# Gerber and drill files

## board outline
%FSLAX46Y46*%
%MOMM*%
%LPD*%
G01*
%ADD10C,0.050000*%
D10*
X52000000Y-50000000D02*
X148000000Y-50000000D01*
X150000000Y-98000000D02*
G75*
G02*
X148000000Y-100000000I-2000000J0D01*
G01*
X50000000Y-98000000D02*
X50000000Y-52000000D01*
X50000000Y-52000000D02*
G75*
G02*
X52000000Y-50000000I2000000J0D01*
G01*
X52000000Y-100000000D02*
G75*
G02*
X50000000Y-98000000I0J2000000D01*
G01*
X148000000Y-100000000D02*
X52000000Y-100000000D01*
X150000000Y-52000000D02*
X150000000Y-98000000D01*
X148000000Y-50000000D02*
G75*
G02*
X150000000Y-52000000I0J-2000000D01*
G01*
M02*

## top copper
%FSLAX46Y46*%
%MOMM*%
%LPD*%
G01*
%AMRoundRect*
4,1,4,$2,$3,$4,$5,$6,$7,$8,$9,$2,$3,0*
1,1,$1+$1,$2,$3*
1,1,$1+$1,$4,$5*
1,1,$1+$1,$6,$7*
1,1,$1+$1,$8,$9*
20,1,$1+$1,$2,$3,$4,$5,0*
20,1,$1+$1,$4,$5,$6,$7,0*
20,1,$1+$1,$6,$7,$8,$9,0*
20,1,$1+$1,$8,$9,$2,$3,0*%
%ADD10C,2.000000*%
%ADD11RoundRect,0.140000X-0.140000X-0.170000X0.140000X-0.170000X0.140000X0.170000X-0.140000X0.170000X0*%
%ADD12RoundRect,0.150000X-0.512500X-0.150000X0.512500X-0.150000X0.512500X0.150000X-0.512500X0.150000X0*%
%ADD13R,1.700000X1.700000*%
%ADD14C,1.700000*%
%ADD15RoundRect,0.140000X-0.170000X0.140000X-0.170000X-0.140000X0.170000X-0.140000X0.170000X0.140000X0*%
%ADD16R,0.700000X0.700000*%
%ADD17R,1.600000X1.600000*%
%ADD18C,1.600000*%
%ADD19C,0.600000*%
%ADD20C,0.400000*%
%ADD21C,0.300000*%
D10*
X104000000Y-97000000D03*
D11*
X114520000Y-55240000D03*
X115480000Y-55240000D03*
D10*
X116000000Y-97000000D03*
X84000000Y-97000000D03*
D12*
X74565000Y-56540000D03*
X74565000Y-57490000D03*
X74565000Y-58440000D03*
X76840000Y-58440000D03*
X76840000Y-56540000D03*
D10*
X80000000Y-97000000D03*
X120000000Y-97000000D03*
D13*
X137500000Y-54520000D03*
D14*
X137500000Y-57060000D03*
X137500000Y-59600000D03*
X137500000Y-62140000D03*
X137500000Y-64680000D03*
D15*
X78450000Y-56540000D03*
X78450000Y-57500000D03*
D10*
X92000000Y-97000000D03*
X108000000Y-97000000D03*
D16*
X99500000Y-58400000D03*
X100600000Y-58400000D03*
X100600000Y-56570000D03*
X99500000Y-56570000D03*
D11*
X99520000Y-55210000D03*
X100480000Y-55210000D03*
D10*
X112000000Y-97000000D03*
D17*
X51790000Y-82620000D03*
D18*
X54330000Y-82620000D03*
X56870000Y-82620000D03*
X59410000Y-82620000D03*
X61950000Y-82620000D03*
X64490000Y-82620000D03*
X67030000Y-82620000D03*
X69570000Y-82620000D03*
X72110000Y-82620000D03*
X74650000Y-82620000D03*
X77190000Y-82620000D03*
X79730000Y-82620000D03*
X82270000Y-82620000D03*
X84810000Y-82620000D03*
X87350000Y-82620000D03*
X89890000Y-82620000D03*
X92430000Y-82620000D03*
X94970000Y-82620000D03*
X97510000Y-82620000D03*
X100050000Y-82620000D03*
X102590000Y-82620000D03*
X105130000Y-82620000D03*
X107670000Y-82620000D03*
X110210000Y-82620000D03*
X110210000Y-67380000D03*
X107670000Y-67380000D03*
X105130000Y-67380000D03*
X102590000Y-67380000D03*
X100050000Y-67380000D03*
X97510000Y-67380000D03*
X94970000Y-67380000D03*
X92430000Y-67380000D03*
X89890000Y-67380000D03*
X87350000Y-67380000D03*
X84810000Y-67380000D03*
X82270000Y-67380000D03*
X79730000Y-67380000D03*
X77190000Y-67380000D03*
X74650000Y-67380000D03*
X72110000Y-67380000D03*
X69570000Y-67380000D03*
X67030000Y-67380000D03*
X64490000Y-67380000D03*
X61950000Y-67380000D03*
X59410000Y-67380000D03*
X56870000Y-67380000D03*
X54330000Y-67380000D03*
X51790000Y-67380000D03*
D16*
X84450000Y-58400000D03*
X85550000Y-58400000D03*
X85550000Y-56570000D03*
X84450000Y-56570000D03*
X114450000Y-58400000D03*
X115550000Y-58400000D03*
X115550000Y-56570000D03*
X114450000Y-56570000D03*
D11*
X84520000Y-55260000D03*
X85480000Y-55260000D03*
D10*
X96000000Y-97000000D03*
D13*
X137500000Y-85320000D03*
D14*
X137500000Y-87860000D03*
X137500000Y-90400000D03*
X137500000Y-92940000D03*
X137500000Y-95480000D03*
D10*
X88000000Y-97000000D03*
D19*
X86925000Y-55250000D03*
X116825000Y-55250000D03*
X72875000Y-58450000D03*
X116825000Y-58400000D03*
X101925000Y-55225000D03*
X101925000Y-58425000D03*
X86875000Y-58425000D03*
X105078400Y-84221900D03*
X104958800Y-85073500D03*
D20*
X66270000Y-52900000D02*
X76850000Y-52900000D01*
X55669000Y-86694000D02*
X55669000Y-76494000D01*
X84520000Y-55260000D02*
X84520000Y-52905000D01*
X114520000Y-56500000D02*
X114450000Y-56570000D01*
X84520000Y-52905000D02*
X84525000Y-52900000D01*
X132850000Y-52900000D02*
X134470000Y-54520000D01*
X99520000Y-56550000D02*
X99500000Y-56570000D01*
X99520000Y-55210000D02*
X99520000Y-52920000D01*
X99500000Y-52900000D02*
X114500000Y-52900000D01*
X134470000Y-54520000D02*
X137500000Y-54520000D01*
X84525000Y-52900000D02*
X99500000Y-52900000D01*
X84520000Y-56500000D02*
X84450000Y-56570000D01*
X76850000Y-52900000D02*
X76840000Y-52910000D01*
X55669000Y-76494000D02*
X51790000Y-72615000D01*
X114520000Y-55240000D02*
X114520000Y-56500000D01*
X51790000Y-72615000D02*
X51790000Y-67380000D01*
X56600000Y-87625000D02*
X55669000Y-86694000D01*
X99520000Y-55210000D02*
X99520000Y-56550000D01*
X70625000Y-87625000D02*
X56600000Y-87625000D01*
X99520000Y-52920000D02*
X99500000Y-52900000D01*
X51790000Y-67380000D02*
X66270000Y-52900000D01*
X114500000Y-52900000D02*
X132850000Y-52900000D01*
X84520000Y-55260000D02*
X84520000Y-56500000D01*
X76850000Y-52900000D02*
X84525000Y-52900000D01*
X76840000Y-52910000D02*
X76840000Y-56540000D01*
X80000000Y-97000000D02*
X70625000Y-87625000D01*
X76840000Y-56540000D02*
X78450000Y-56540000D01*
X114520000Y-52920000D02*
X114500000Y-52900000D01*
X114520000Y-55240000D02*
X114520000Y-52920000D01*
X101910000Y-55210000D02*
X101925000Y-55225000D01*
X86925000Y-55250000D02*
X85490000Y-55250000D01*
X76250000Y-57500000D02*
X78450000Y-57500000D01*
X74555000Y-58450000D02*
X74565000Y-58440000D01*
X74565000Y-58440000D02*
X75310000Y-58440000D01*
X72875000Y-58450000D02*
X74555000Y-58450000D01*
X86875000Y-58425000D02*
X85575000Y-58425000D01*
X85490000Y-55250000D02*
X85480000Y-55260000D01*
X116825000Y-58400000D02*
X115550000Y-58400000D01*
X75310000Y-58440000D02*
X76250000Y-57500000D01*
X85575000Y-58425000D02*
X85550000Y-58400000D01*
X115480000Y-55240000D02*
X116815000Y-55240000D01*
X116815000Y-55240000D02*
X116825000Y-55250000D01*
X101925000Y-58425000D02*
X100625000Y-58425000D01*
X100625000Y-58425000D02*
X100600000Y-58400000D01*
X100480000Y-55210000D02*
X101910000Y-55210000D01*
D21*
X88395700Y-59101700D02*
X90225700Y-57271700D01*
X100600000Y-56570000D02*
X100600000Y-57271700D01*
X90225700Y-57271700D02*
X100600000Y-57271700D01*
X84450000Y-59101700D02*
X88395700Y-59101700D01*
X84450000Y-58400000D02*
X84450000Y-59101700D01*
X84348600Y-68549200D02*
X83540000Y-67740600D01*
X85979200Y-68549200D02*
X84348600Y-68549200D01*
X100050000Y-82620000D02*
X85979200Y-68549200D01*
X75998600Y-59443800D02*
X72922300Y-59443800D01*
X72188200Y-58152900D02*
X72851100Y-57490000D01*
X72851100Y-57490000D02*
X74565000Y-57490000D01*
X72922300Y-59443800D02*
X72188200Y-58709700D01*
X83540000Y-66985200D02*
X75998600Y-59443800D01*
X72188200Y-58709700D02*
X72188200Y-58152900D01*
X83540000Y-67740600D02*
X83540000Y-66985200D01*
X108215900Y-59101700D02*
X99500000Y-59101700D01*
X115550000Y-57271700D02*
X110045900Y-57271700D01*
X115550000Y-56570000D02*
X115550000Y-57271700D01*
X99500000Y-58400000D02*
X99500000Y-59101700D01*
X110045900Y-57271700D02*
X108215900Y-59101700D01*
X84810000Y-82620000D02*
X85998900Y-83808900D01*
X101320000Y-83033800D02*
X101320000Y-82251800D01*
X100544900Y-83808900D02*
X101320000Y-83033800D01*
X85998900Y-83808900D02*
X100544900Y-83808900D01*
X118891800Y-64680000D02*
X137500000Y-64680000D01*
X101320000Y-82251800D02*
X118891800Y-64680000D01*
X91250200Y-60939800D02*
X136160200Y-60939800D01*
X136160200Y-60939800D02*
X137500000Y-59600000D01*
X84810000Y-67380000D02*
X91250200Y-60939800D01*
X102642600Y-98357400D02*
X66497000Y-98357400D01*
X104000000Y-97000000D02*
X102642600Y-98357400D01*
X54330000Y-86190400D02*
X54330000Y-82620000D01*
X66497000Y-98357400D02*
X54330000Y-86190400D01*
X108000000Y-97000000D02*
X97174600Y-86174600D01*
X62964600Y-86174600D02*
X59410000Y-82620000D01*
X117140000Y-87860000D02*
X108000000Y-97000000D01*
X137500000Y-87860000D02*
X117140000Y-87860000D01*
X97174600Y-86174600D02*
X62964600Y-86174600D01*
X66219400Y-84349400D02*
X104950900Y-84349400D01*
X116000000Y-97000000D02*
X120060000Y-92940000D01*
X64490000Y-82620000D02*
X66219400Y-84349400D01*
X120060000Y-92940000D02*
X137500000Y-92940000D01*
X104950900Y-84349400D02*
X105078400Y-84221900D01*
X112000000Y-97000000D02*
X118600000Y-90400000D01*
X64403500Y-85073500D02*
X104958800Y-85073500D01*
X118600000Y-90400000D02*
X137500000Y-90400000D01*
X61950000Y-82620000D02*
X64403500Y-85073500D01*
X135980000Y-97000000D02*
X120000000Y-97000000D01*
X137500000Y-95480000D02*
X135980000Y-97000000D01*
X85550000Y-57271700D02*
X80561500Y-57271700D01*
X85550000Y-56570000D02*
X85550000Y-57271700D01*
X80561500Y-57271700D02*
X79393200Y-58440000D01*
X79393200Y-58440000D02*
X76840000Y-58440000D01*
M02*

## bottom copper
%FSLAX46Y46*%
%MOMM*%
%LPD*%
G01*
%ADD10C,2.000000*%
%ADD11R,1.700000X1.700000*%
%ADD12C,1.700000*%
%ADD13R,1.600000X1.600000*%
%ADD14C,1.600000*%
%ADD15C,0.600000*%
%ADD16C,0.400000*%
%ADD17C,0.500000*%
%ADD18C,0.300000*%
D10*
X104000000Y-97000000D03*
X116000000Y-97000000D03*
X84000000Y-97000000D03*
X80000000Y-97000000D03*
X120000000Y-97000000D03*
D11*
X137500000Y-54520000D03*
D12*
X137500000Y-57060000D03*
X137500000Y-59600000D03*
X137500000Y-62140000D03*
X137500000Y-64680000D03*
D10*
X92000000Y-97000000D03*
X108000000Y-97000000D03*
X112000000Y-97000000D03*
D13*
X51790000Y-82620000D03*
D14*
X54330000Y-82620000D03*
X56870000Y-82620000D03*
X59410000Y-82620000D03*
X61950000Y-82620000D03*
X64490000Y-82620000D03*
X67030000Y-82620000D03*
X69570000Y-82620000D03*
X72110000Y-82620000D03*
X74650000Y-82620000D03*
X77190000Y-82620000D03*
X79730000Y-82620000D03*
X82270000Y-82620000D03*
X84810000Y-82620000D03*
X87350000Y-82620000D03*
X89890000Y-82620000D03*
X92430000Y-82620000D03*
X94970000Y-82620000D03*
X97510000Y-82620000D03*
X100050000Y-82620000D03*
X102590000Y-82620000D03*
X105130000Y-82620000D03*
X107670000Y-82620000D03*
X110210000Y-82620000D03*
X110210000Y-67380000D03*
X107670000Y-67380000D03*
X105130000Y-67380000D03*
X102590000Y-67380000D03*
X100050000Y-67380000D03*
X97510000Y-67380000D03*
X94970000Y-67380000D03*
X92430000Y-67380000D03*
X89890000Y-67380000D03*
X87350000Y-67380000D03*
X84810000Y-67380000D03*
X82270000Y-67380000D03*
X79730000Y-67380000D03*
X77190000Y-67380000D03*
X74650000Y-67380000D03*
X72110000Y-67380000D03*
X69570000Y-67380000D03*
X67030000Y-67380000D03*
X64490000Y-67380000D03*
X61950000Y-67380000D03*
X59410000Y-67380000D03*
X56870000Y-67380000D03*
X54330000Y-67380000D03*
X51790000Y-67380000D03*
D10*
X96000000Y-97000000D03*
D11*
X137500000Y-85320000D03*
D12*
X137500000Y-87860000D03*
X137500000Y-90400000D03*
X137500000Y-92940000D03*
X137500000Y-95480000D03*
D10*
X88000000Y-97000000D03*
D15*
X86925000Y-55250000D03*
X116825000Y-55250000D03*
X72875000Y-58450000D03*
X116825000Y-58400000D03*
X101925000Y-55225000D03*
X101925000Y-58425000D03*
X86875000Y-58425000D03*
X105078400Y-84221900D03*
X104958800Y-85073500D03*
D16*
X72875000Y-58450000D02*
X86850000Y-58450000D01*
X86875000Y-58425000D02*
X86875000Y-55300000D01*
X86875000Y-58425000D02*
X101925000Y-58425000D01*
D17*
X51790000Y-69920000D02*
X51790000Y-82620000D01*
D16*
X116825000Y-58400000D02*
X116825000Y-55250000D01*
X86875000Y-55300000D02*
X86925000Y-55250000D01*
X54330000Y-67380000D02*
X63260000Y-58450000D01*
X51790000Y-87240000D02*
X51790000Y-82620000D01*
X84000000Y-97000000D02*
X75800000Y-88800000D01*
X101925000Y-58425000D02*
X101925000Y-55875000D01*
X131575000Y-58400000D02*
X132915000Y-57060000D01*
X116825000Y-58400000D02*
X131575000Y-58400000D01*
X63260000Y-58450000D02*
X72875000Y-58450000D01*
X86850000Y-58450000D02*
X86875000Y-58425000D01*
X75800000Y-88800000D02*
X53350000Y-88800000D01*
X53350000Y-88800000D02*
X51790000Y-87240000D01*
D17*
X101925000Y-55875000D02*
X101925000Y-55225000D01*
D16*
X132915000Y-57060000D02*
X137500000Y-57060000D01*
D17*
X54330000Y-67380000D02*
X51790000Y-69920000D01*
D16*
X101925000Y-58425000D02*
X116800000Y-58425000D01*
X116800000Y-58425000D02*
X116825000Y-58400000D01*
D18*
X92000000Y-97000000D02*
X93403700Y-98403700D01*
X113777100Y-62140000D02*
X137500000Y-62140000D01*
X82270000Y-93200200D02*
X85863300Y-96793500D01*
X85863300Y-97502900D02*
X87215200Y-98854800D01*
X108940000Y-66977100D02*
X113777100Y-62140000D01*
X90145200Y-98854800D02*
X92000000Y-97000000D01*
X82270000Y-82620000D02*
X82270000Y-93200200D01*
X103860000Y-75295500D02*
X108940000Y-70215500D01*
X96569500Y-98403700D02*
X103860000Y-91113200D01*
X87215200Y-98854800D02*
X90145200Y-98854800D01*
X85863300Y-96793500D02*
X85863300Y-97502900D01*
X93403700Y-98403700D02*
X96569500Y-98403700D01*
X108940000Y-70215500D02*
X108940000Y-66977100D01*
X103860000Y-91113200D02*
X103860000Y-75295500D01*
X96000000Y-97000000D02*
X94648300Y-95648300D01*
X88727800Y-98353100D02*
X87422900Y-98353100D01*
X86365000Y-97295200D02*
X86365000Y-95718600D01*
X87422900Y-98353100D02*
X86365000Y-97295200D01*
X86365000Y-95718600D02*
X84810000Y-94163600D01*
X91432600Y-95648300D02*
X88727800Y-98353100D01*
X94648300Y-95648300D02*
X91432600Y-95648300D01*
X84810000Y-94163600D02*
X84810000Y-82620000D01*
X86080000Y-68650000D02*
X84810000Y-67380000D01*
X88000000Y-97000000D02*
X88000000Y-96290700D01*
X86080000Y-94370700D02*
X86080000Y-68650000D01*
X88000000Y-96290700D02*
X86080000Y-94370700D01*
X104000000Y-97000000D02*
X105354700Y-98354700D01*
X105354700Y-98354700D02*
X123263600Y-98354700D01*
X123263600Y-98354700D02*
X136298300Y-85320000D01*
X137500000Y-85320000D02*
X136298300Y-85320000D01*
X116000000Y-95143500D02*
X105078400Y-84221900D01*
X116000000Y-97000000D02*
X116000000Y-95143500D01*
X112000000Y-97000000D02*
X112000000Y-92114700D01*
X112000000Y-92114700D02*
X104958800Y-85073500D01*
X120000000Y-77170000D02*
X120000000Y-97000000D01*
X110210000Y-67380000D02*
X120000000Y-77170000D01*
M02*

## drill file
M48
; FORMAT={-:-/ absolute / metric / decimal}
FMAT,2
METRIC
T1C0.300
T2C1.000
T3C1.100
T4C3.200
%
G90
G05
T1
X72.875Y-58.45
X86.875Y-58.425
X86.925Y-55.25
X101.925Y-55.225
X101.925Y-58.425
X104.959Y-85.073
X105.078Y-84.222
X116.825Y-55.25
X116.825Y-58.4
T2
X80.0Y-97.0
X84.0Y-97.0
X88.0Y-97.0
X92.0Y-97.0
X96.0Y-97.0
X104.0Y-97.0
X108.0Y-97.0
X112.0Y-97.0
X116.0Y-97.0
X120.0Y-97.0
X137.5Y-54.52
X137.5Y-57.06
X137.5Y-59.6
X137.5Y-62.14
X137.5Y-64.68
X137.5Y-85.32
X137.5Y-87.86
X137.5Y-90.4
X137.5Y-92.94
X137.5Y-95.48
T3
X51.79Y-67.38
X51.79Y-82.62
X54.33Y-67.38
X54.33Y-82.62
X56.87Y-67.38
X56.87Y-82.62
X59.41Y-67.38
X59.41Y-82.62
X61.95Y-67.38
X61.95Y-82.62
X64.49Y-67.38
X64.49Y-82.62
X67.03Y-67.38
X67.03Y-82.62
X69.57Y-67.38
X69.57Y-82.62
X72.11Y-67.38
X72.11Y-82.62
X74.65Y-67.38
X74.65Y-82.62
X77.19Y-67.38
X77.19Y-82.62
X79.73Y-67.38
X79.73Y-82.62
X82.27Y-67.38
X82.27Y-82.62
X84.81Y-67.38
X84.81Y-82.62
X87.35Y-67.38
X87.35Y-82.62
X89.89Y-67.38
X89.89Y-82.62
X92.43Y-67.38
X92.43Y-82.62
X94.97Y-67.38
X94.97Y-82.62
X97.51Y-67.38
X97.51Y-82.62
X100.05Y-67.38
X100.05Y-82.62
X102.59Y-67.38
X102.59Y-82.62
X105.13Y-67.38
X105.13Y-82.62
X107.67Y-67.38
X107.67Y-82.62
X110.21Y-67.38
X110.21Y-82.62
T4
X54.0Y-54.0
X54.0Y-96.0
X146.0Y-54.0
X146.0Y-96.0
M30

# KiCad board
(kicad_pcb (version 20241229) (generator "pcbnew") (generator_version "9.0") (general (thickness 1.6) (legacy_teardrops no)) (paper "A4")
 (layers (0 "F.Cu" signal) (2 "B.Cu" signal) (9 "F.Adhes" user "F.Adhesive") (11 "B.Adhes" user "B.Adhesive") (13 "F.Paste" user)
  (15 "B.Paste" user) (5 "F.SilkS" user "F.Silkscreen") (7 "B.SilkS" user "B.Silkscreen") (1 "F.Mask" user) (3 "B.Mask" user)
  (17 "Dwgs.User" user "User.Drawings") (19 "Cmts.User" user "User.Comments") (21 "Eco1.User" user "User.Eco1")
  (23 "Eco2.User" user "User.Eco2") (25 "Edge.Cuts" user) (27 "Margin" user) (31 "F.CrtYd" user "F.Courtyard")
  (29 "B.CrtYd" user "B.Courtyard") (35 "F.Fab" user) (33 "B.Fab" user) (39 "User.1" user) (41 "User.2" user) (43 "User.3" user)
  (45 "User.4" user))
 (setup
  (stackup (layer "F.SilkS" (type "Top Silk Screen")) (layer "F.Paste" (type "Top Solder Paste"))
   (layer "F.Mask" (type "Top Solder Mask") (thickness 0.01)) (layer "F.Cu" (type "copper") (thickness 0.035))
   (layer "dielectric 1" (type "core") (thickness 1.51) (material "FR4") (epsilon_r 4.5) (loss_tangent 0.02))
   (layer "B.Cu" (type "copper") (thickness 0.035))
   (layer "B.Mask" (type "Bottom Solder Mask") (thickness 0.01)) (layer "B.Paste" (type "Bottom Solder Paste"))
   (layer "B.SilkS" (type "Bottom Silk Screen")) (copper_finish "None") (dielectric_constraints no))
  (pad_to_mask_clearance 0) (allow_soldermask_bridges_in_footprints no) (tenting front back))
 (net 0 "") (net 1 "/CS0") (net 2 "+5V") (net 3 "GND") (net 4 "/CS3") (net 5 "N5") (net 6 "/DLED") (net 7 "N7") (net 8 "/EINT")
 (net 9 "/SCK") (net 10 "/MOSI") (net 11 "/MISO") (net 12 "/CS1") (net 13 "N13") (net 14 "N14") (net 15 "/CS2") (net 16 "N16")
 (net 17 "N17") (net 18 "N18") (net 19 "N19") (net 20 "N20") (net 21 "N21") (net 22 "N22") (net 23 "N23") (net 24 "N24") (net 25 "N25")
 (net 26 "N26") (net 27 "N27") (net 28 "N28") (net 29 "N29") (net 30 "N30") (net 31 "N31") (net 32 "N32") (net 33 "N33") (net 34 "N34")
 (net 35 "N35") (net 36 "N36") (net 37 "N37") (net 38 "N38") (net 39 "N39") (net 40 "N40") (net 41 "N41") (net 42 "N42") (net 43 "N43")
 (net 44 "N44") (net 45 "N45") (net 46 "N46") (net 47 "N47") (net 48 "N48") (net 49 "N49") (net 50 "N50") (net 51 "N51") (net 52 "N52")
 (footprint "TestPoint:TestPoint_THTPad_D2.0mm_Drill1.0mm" (layer "F.Cu") (at 104 97 90)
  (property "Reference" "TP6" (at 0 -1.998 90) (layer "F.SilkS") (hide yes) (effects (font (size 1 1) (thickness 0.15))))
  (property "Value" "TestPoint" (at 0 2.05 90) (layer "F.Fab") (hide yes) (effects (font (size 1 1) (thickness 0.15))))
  (pad "1" thru_hole circle (at 0 0 90) (size 2 2) (drill 1) (layers "*.Cu" "*.Mask") (remove_unused_layers no) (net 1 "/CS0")))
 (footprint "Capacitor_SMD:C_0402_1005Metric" (layer "F.Cu") (at 115 55.24)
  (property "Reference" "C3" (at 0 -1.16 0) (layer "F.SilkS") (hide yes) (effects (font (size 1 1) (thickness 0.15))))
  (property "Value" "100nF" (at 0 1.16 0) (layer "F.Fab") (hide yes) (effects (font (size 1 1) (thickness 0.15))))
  (pad "1" smd roundrect (at -0.48 0) (size 0.56 0.62) (layers "F.Cu" "F.Mask" "F.Paste") (roundrect_rratio 0.25) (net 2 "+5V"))
  (pad "2" smd roundrect (at 0.48 0) (size 0.56 0.62) (layers "F.Cu" "F.Mask" "F.Paste") (roundrect_rratio 0.25) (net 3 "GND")))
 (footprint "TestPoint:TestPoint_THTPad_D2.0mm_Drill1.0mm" (layer "F.Cu") (at 116 97 90)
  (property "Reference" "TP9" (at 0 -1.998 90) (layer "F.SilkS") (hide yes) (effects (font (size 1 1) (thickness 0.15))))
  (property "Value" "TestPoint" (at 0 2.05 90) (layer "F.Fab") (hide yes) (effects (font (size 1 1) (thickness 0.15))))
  (pad "1" thru_hole circle (at 0 0 90) (size 2 2) (drill 1) (layers "*.Cu" "*.Mask") (remove_unused_layers no) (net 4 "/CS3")))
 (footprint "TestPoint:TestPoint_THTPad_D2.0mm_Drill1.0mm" (layer "F.Cu") (at 84 97 90)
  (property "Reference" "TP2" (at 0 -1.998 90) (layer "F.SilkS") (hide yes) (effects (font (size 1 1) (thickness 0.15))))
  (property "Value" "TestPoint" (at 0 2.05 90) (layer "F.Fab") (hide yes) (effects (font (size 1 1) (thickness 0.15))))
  (pad "1" thru_hole circle (at 0 0 90) (size 2 2) (drill 1) (layers "*.Cu" "*.Mask") (remove_unused_layers no) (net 3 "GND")))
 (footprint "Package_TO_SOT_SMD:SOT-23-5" (layer "F.Cu") (at 75.7025 57.49)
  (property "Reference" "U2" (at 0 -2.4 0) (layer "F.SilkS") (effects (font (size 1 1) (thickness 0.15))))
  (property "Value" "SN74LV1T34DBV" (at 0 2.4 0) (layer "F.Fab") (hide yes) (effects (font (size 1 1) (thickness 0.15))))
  (pad "1" smd roundrect (at -1.1375 -0.95) (size 1.325 0.6) (layers "F.Cu" "F.Mask" "F.Paste") (roundrect_rratio 0.25) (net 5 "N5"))
  (pad "2" smd roundrect (at -1.1375 0) (size 1.325 0.6) (layers "F.Cu" "F.Mask" "F.Paste") (roundrect_rratio 0.25) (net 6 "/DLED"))
  (pad "3" smd roundrect (at -1.1375 0.95) (size 1.325 0.6) (layers "F.Cu" "F.Mask" "F.Paste") (roundrect_rratio 0.25) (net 3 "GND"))
  (pad "4" smd roundrect (at 1.1375 0.95) (size 1.325 0.6) (layers "F.Cu" "F.Mask" "F.Paste") (roundrect_rratio 0.25) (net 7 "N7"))
  (pad "5" smd roundrect (at 1.1375 -0.95) (size 1.325 0.6) (layers "F.Cu" "F.Mask" "F.Paste") (roundrect_rratio 0.25) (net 2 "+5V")))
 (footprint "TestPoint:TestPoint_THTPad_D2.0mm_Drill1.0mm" (layer "F.Cu") (at 80 97 90)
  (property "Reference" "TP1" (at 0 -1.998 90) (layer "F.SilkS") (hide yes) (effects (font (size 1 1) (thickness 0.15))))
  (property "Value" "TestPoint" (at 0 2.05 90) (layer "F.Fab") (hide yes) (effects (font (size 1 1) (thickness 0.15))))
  (pad "1" thru_hole circle (at 0 0 90) (size 2 2) (drill 1) (layers "*.Cu" "*.Mask") (remove_unused_layers no) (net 2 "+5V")))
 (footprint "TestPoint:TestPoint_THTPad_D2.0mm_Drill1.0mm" (layer "F.Cu") (at 120 97 90)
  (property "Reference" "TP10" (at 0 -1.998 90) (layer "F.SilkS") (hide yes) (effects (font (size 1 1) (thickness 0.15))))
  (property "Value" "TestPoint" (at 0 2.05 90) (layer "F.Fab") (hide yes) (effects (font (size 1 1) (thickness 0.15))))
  (pad "1" thru_hole circle (at 0 0 90) (size 2 2) (drill 1) (layers "*.Cu" "*.Mask") (remove_unused_layers no) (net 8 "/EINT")))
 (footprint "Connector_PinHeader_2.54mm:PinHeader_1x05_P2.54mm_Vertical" (layer "F.Cu") (at 137.5 54.52)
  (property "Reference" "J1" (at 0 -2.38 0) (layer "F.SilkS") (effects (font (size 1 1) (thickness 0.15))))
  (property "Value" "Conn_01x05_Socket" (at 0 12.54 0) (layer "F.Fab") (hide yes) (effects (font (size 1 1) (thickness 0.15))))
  (pad "1" thru_hole rect (at 0 0) (size 1.7 1.7) (drill 1) (layers "*.Cu" "*.Mask") (remove_unused_layers no) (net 2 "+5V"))
  (pad "2" thru_hole circle (at 0 2.54) (size 1.7 1.7) (drill 1) (layers "*.Cu" "*.Mask") (remove_unused_layers no) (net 3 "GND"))
  (pad "3" thru_hole circle (at 0 5.08) (size 1.7 1.7) (drill 1) (layers "*.Cu" "*.Mask") (remove_unused_layers no) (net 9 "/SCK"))
  (pad "4" thru_hole circle (at 0 7.62) (size 1.7 1.7) (drill 1) (layers "*.Cu" "*.Mask") (remove_unused_layers no) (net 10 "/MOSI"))
  (pad "5" thru_hole circle (at 0 10.16) (size 1.7 1.7) (drill 1) (layers "*.Cu" "*.Mask") (remove_unused_layers no) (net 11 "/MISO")))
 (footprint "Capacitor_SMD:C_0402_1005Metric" (layer "F.Cu") (at 78.45 57.02 -90)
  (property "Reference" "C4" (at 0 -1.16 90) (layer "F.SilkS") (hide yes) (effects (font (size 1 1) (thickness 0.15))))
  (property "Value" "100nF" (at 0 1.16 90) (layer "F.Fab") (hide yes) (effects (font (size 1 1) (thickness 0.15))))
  (pad "1" smd roundrect (at -0.48 0 270) (size 0.56 0.62) (layers "F.Cu" "F.Mask" "F.Paste") (roundrect_rratio 0.25) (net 2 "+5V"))
  (pad "2" smd roundrect (at 0.48 0 270) (size 0.56 0.62) (layers "F.Cu" "F.Mask" "F.Paste") (roundrect_rratio 0.25) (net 3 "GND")))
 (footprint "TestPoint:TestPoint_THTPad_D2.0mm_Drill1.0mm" (layer "F.Cu") (at 92 97 90)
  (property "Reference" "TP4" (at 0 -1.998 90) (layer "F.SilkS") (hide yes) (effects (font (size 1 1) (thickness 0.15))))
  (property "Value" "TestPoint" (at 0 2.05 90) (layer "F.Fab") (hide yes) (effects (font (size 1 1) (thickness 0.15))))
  (pad "1" thru_hole circle (at 0 0 90) (size 2 2) (drill 1) (layers "*.Cu" "*.Mask") (remove_unused_layers no) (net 10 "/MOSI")))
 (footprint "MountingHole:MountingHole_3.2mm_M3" (layer "F.Cu") (at 54 96)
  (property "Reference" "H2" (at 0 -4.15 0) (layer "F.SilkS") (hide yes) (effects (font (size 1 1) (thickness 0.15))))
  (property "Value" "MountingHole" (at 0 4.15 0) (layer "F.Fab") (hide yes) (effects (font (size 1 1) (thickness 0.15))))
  (pad "" np_thru_hole circle (at 0 0) (size 3.2 3.2) (drill 3.2) (layers "*.Cu" "*.Mask")))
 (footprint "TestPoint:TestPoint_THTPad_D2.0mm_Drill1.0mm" (layer "F.Cu") (at 108 97 90)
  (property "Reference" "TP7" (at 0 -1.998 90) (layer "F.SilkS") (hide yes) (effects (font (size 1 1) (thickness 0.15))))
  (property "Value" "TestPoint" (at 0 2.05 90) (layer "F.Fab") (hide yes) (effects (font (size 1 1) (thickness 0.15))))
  (pad "1" thru_hole circle (at 0 0 90) (size 2 2) (drill 1) (layers "*.Cu" "*.Mask") (remove_unused_layers no) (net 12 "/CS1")))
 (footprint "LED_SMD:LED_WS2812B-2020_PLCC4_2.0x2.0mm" (layer "F.Cu") (at 100.05 57.485 90)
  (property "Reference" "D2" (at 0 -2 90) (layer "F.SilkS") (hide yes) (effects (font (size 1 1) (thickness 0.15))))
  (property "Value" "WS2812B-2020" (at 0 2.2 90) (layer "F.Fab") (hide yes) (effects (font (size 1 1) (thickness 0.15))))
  (pad "1" smd rect (at -0.915 -0.55 90) (size 0.7 0.7) (layers "F.Cu" "F.Mask" "F.Paste") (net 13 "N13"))
  (pad "2" smd rect (at -0.915 0.55 90) (size 0.7 0.7) (layers "F.Cu" "F.Mask" "F.Paste") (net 3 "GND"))
  (pad "3" smd rect (at 0.915 0.55 90) (size 0.7 0.7) (layers "F.Cu" "F.Mask" "F.Paste") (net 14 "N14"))
  (pad "4" smd rect (at 0.915 -0.55 90) (size 0.7 0.7) (layers "F.Cu" "F.Mask" "F.Paste") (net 2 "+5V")))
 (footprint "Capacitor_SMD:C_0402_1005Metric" (layer "F.Cu") (at 100 55.21)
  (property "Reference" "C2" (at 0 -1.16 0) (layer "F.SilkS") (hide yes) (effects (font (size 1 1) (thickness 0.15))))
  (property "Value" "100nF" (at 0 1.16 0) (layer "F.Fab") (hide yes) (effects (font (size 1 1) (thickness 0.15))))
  (pad "1" smd roundrect (at -0.48 0) (size 0.56 0.62) (layers "F.Cu" "F.Mask" "F.Paste") (roundrect_rratio 0.25) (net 2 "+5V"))
  (pad "2" smd roundrect (at 0.48 0) (size 0.56 0.62) (layers "F.Cu" "F.Mask" "F.Paste") (roundrect_rratio 0.25) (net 3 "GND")))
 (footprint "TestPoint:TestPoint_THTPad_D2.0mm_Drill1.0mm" (layer "F.Cu") (at 112 97 90)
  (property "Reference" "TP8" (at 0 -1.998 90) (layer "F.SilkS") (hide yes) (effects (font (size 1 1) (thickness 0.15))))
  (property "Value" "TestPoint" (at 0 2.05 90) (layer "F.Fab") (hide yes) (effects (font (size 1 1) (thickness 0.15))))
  (pad "1" thru_hole circle (at 0 0 90) (size 2 2) (drill 1) (layers "*.Cu" "*.Mask") (remove_unused_layers no) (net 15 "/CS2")))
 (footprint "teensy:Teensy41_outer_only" (layer "F.Cu") (at 81 75)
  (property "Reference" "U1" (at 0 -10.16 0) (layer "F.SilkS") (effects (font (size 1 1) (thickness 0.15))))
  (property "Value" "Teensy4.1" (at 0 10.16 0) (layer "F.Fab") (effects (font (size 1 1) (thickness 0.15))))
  (pad "1" thru_hole rect (at -29.21 7.62) (size 1.6 1.6) (drill 1.1) (layers "*.Cu" "*.Mask") (remove_unused_layers no) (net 3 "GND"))
  (pad "2" thru_hole circle (at -26.67 7.62) (size 1.6 1.6) (drill 1.1) (layers "*.Cu" "*.Mask") (remove_unused_layers no) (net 1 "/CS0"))
  (pad "3" thru_hole circle (at -24.13 7.62) (size 1.6 1.6) (drill 1.1) (layers "*.Cu" "*.Mask") (remove_unused_layers no) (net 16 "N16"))
  (pad "4" thru_hole circle (at -21.59 7.62) (size 1.6 1.6) (drill 1.1) (layers "*.Cu" "*.Mask") (remove_unused_layers no) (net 12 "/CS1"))
  (pad "5" thru_hole circle (at -19.05 7.62) (size 1.6 1.6) (drill 1.1) (layers "*.Cu" "*.Mask") (remove_unused_layers no) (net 15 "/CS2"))
  (pad "6" thru_hole circle (at -16.51 7.62) (size 1.6 1.6) (drill 1.1) (layers "*.Cu" "*.Mask") (remove_unused_layers no) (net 4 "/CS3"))
  (pad "7" thru_hole circle (at -13.97 7.62) (size 1.6 1.6) (drill 1.1) (layers "*.Cu" "*.Mask") (remove_unused_layers no) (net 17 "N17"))
  (pad "8" thru_hole circle (at -11.43 7.62) (size 1.6 1.6) (drill 1.1) (layers "*.Cu" "*.Mask") (remove_unused_layers no) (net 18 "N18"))
  (pad "9" thru_hole circle (at -8.89 7.62) (size 1.6 1.6) (drill 1.1) (layers "*.Cu" "*.Mask") (remove_unused_layers no) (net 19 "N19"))
  (pad "10" thru_hole circle (at -6.35 7.62) (size 1.6 1.6) (drill 1.1) (layers "*.Cu" "*.Mask") (remove_unused_layers no) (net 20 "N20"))
  (pad "11" thru_hole circle (at -3.81 7.62) (size 1.6 1.6) (drill 1.1) (layers "*.Cu" "*.Mask") (remove_unused_layers no) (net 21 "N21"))
  (pad "12" thru_hole circle (at -1.27 7.62) (size 1.6 1.6) (drill 1.1) (layers "*.Cu" "*.Mask") (remove_unused_layers no) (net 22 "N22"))
  (pad "13" thru_hole circle (at 1.27 7.62) (size 1.6 1.6) (drill 1.1) (layers "*.Cu" "*.Mask") (remove_unused_layers no) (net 10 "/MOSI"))
  (pad "14" thru_hole circle (at 3.81 7.62) (size 1.6 1.6) (drill 1.1) (layers "*.Cu" "*.Mask") (remove_unused_layers no) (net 11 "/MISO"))
  (pad "15" thru_hole circle (at 6.35 7.62) (size 1.6 1.6) (drill 1.1) (layers "*.Cu" "*.Mask") (remove_unused_layers no) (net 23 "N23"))
  (pad "16" thru_hole circle (at 8.89 7.62) (size 1.6 1.6) (drill 1.1) (layers "*.Cu" "*.Mask") (remove_unused_layers no) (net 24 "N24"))
  (pad "17" thru_hole circle (at 11.43 7.62) (size 1.6 1.6) (drill 1.1) (layers "*.Cu" "*.Mask") (remove_unused_layers no) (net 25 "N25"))
  (pad "18" thru_hole circle (at 13.97 7.62) (size 1.6 1.6) (drill 1.1) (layers "*.Cu" "*.Mask") (remove_unused_layers no) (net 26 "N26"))
  (pad "19" thru_hole circle (at 16.51 7.62) (size 1.6 1.6) (drill 1.1) (layers "*.Cu" "*.Mask") (remove_unused_layers no) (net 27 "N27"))
  (pad "20" thru_hole circle (at 19.05 7.62) (size 1.6 1.6) (drill 1.1) (layers "*.Cu" "*.Mask") (remove_unused_layers no) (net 6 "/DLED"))
  (pad "21" thru_hole circle (at 21.59 7.62) (size 1.6 1.6) (drill 1.1) (layers "*.Cu" "*.Mask") (remove_unused_layers no) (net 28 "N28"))
  (pad "22" thru_hole circle (at 24.13 7.62) (size 1.6 1.6) (drill 1.1) (layers "*.Cu" "*.Mask") (remove_unused_layers no) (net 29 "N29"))
  (pad "23" thru_hole circle (at 26.67 7.62) (size 1.6 1.6) (drill 1.1) (layers "*.Cu" "*.Mask") (remove_unused_layers no) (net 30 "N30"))
  (pad "24" thru_hole circle (at 29.21 7.62) (size 1.6 1.6) (drill 1.1) (layers "*.Cu" "*.Mask") (remove_unused_layers no) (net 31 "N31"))
  (pad "25" thru_hole circle (at 29.21 -7.62) (size 1.6 1.6) (drill 1.1) (layers "*.Cu" "*.Mask") (remove_unused_layers no) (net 8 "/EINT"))
  (pad "26" thru_hole circle (at 26.67 -7.62) (size 1.6 1.6) (drill 1.1) (layers "*.Cu" "*.Mask") (remove_unused_layers no) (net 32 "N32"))
  (pad "27" thru_hole circle (at 24.13 -7.62) (size 1.6 1.6) (drill 1.1) (layers "*.Cu" "*.Mask") (remove_unused_layers no) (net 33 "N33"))
  (pad "28" thru_hole circle (at 21.59 -7.62) (size 1.6 1.6) (drill 1.1) (layers "*.Cu" "*.Mask") (remove_unused_layers no) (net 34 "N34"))
  (pad "29" thru_hole circle (at 19.05 -7.62) (size 1.6 1.6) (drill 1.1) (layers "*.Cu" "*.Mask") (remove_unused_layers no) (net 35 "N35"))
  (pad "30" thru_hole circle (at 16.51 -7.62) (size 1.6 1.6) (drill 1.1) (layers "*.Cu" "*.Mask") (remove_unused_layers no) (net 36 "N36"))
  (pad "31" thru_hole circle (at 13.97 -7.62) (size 1.6 1.6) (drill 1.1) (layers "*.Cu" "*.Mask") (remove_unused_layers no) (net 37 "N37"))
  (pad "32" thru_hole circle (at 11.43 -7.62) (size 1.6 1.6) (drill 1.1) (layers "*.Cu" "*.Mask") (remove_unused_layers no) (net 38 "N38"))
  (pad "33" thru_hole circle (at 8.89 -7.62) (size 1.6 1.6) (drill 1.1) (layers "*.Cu" "*.Mask") (remove_unused_layers no) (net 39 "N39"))
  (pad "34" thru_hole circle (at 6.35 -7.62) (size 1.6 1.6) (drill 1.1) (layers "*.Cu" "*.Mask") (remove_unused_layers no) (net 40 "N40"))
  (pad "35" thru_hole circle (at 3.81 -7.62) (size 1.6 1.6) (drill 1.1) (layers "*.Cu" "*.Mask") (remove_unused_layers no) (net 9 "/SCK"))
  (pad "36" thru_hole circle (at 1.27 -7.62) (size 1.6 1.6) (drill 1.1) (layers "*.Cu" "*.Mask") (remove_unused_layers no) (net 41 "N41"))
  (pad "37" thru_hole circle (at -1.27 -7.62) (size 1.6 1.6) (drill 1.1) (layers "*.Cu" "*.Mask") (remove_unused_layers no) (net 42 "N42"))
  (pad "38" thru_hole circle (at -3.81 -7.62) (size 1.6 1.6) (drill 1.1) (layers "*.Cu" "*.Mask") (remove_unused_layers no) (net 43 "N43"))
  (pad "39" thru_hole circle (at -6.35 -7.62) (size 1.6 1.6) (drill 1.1) (layers "*.Cu" "*.Mask") (remove_unused_layers no) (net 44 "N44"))
  (pad "40" thru_hole circle (at -8.89 -7.62) (size 1.6 1.6) (drill 1.1) (layers "*.Cu" "*.Mask") (remove_unused_layers no) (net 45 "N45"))
  (pad "41" thru_hole circle (at -11.43 -7.62) (size 1.6 1.6) (drill 1.1) (layers "*.Cu" "*.Mask") (remove_unused_layers no) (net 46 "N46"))
  (pad "42" thru_hole circle (at -13.97 -7.62) (size 1.6 1.6) (drill 1.1) (layers "*.Cu" "*.Mask") (remove_unused_layers no) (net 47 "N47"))
  (pad "43" thru_hole circle (at -16.51 -7.62) (size 1.6 1.6) (drill 1.1) (layers "*.Cu" "*.Mask") (remove_unused_layers no) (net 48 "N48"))
  (pad "44" thru_hole circle (at -19.05 -7.62) (size 1.6 1.6) (drill 1.1) (layers "*.Cu" "*.Mask") (remove_unused_layers no) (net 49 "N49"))
  (pad "45" thru_hole circle (at -21.59 -7.62) (size 1.6 1.6) (drill 1.1) (layers "*.Cu" "*.Mask") (remove_unused_layers no) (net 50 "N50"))
  (pad "46" thru_hole circle (at -24.13 -7.62) (size 1.6 1.6) (drill 1.1) (layers "*.Cu" "*.Mask") (remove_unused_layers no) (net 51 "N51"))
  (pad "47" thru_hole circle (at -26.67 -7.62) (size 1.6 1.6) (drill 1.1) (layers "*.Cu" "*.Mask") (remove_unused_layers no) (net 3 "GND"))
  (pad "48" thru_hole circle (at -29.21 -7.62) (size 1.6 1.6) (drill 1.1) (layers "*.Cu" "*.Mask") (remove_unused_layers no) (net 2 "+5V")))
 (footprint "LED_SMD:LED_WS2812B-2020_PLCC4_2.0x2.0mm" (layer "F.Cu") (at 85 57.485 90)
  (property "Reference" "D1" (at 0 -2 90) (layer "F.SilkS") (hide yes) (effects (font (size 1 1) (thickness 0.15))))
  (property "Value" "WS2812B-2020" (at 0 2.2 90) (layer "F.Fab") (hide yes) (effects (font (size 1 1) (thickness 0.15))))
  (pad "1" smd rect (at -0.915 -0.55 90) (size 0.7 0.7) (layers "F.Cu" "F.Mask" "F.Paste") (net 14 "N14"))
  (pad "2" smd rect (at -0.915 0.55 90) (size 0.7 0.7) (layers "F.Cu" "F.Mask" "F.Paste") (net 3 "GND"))
  (pad "3" smd rect (at 0.915 0.55 90) (size 0.7 0.7) (layers "F.Cu" "F.Mask" "F.Paste") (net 7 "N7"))
  (pad "4" smd rect (at 0.915 -0.55 90) (size 0.7 0.7) (layers "F.Cu" "F.Mask" "F.Paste") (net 2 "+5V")))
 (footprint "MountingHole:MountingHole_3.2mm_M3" (layer "F.Cu") (at 146 96)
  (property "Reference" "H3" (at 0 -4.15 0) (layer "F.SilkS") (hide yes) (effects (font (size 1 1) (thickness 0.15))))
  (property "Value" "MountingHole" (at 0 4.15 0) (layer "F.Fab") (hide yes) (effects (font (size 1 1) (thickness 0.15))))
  (pad "" np_thru_hole circle (at 0 0) (size 3.2 3.2) (drill 3.2) (layers "*.Cu" "*.Mask")))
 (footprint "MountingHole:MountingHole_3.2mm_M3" (layer "F.Cu") (at 146 54)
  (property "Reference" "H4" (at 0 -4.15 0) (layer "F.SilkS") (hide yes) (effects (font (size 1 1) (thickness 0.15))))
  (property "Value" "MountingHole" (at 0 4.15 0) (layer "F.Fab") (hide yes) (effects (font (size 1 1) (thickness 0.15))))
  (pad "" np_thru_hole circle (at 0 0) (size 3.2 3.2) (drill 3.2) (layers "*.Cu" "*.Mask")))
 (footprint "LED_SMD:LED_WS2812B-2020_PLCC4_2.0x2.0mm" (layer "F.Cu") (at 115 57.485 90)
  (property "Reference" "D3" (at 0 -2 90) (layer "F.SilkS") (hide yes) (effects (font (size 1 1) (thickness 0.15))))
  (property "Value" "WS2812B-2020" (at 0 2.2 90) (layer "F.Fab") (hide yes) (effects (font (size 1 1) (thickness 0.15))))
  (pad "1" smd rect (at -0.915 -0.55 90) (size 0.7 0.7) (layers "F.Cu" "F.Mask" "F.Paste") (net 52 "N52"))
  (pad "2" smd rect (at -0.915 0.55 90) (size 0.7 0.7) (layers "F.Cu" "F.Mask" "F.Paste") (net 3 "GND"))
  (pad "3" smd rect (at 0.915 0.55 90) (size 0.7 0.7) (layers "F.Cu" "F.Mask" "F.Paste") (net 13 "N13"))
  (pad "4" smd rect (at 0.915 -0.55 90) (size 0.7 0.7) (layers "F.Cu" "F.Mask" "F.Paste") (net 2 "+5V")))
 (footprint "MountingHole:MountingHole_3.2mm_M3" (layer "F.Cu") (at 54 54)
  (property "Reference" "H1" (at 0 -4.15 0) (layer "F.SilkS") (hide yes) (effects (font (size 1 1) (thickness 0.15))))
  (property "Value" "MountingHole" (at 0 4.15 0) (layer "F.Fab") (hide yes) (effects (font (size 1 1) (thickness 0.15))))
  (pad "" np_thru_hole circle (at 0 0) (size 3.2 3.2) (drill 3.2) (layers "*.Cu" "*.Mask")))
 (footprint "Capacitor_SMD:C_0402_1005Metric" (layer "F.Cu") (at 85 55.26)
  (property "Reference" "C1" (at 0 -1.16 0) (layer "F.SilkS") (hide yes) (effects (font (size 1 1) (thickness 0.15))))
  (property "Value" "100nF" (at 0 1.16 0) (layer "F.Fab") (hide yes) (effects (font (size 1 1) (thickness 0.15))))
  (pad "1" smd roundrect (at -0.48 0) (size 0.56 0.62) (layers "F.Cu" "F.Mask" "F.Paste") (roundrect_rratio 0.25) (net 2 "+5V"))
  (pad "2" smd roundrect (at 0.48 0) (size 0.56 0.62) (layers "F.Cu" "F.Mask" "F.Paste") (roundrect_rratio 0.25) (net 3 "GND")))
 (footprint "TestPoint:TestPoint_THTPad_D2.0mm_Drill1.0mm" (layer "F.Cu") (at 96 97 90)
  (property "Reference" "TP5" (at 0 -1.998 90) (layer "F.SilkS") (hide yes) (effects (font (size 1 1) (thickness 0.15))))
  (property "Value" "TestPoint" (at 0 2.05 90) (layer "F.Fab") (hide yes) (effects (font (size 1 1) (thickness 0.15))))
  (pad "1" thru_hole circle (at 0 0 90) (size 2 2) (drill 1) (layers "*.Cu" "*.Mask") (remove_unused_layers no) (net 11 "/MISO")))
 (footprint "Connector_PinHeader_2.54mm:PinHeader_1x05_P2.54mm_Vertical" (layer "F.Cu") (at 137.5 85.32)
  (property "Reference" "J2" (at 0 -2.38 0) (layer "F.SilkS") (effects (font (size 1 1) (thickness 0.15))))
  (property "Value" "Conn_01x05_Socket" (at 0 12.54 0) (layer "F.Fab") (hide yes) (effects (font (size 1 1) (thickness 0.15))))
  (pad "1" thru_hole rect (at 0 0) (size 1.7 1.7) (drill 1) (layers "*.Cu" "*.Mask") (remove_unused_layers no) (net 1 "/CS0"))
  (pad "2" thru_hole circle (at 0 2.54) (size 1.7 1.7) (drill 1) (layers "*.Cu" "*.Mask") (remove_unused_layers no) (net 12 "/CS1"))
  (pad "3" thru_hole circle (at 0 5.08) (size 1.7 1.7) (drill 1) (layers "*.Cu" "*.Mask") (remove_unused_layers no) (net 15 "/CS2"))
  (pad "4" thru_hole circle (at 0 7.62) (size 1.7 1.7) (drill 1) (layers "*.Cu" "*.Mask") (remove_unused_layers no) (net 4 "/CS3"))
  (pad "5" thru_hole circle (at 0 10.16) (size 1.7 1.7) (drill 1) (layers "*.Cu" "*.Mask") (remove_unused_layers no) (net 8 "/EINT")))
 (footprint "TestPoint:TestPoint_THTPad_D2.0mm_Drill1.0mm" (layer "F.Cu") (at 88 97 90)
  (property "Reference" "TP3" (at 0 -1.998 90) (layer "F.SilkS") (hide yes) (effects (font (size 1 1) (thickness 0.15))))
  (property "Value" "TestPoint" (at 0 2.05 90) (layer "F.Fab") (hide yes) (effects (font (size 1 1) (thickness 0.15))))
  (pad "1" thru_hole circle (at 0 0 90) (size 2 2) (drill 1) (layers "*.Cu" "*.Mask") (remove_unused_layers no) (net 9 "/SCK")))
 (gr_line (start 52 50) (end 148 50) (stroke (width 0.05) (type default)) (layer "Edge.Cuts"))
 (gr_arc (start 150 98) (mid 149.414214 99.414214) (end 148 100) (stroke (width 0.05) (type default)) (layer "Edge.Cuts"))
 (gr_line (start 50 98) (end 50 52) (stroke (width 0.05) (type default)) (layer "Edge.Cuts"))
 (gr_arc (start 50 52) (mid 50.585786 50.585786) (end 52 50) (stroke (width 0.05) (type default)) (layer "Edge.Cuts"))
 (gr_arc (start 52 100) (mid 50.585786 99.414214) (end 50 98) (stroke (width 0.05) (type default)) (layer "Edge.Cuts"))
 (gr_line (start 148 100) (end 52 100) (stroke (width 0.05) (type default)) (layer "Edge.Cuts"))
 (gr_line (start 150 52) (end 150 98) (stroke (width 0.05) (type default)) (layer "Edge.Cuts"))
 (gr_arc (start 148 50) (mid 149.414214 50.585786) (end 150 52) (stroke (width 0.05) (type default)) (layer "Edge.Cuts"))
 (segment (start 66.27 52.9) (end 76.85 52.9) (width 0.4) (layer "F.Cu") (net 2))
 (segment (start 55.669 86.694) (end 55.669 76.494) (width 0.4) (layer "F.Cu") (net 2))
 (segment (start 84.52 55.26) (end 84.52 52.905) (width 0.4) (layer "F.Cu") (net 2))
 (segment (start 114.52 56.5) (end 114.45 56.57) (width 0.4) (layer "F.Cu") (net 2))
 (segment (start 84.52 52.905) (end 84.525 52.9) (width 0.4) (layer "F.Cu") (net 2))
 (segment (start 132.85 52.9) (end 134.47 54.52) (width 0.4) (layer "F.Cu") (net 2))
 (segment (start 99.52 56.55) (end 99.5 56.57) (width 0.4) (layer "F.Cu") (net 2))
 (segment (start 99.52 55.21) (end 99.52 52.92) (width 0.4) (layer "F.Cu") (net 2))
 (segment (start 99.5 52.9) (end 114.5 52.9) (width 0.4) (layer "F.Cu") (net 2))
 (segment (start 134.47 54.52) (end 137.5 54.52) (width 0.4) (layer "F.Cu") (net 2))
 (segment (start 84.525 52.9) (end 99.5 52.9) (width 0.4) (layer "F.Cu") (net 2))
 (segment (start 84.52 56.5) (end 84.45 56.57) (width 0.4) (layer "F.Cu") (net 2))
 (segment (start 76.85 52.9) (end 76.84 52.91) (width 0.4) (layer "F.Cu") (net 2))
 (segment (start 55.669 76.494) (end 51.79 72.615) (width 0.4) (layer "F.Cu") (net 2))
 (segment (start 114.52 55.24) (end 114.52 56.5) (width 0.4) (layer "F.Cu") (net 2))
 (segment (start 51.79 72.615) (end 51.79 67.38) (width 0.4) (layer "F.Cu") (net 2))
 (segment (start 56.6 87.625) (end 55.669 86.694) (width 0.4) (layer "F.Cu") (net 2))
 (segment (start 99.52 55.21) (end 99.52 56.55) (width 0.4) (layer "F.Cu") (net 2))
 (segment (start 70.625 87.625) (end 56.6 87.625) (width 0.4) (layer "F.Cu") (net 2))
 (segment (start 99.52 52.92) (end 99.5 52.9) (width 0.4) (layer "F.Cu") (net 2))
 (segment (start 51.79 67.38) (end 66.27 52.9) (width 0.4) (layer "F.Cu") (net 2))
 (segment (start 114.5 52.9) (end 132.85 52.9) (width 0.4) (layer "F.Cu") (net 2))
 (segment (start 84.52 55.26) (end 84.52 56.5) (width 0.4) (layer "F.Cu") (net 2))
 (segment (start 76.85 52.9) (end 84.525 52.9) (width 0.4) (layer "F.Cu") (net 2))
 (segment (start 76.84 52.91) (end 76.84 56.54) (width 0.4) (layer "F.Cu") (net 2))
 (segment (start 80 97) (end 70.625 87.625) (width 0.4) (layer "F.Cu") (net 2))
 (segment (start 76.84 56.54) (end 78.45 56.54) (width 0.4) (layer "F.Cu") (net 2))
 (segment (start 114.52 52.92) (end 114.5 52.9) (width 0.4) (layer "F.Cu") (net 2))
 (segment (start 114.52 55.24) (end 114.52 52.92) (width 0.4) (layer "F.Cu") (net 2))
 (segment (start 101.91 55.21) (end 101.925 55.225) (width 0.4) (layer "F.Cu") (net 3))
 (segment (start 86.925 55.25) (end 85.49 55.25) (width 0.4) (layer "F.Cu") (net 3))
 (segment (start 76.25 57.5) (end 78.45 57.5) (width 0.4) (layer "F.Cu") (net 3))
 (segment (start 74.555 58.45) (end 74.565 58.44) (width 0.4) (layer "F.Cu") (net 3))
 (segment (start 74.565 58.44) (end 75.31 58.44) (width 0.4) (layer "F.Cu") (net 3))
 (segment (start 72.875 58.45) (end 74.555 58.45) (width 0.4) (layer "F.Cu") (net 3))
 (segment (start 86.875 58.425) (end 85.575 58.425) (width 0.4) (layer "F.Cu") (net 3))
 (segment (start 85.49 55.25) (end 85.48 55.26) (width 0.4) (layer "F.Cu") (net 3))
 (segment (start 116.825 58.4) (end 115.55 58.4) (width 0.4) (layer "F.Cu") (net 3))
 (segment (start 75.31 58.44) (end 76.25 57.5) (width 0.4) (layer "F.Cu") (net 3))
 (segment (start 85.575 58.425) (end 85.55 58.4) (width 0.4) (layer "F.Cu") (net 3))
 (segment (start 115.48 55.24) (end 116.815 55.24) (width 0.4) (layer "F.Cu") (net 3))
 (segment (start 116.815 55.24) (end 116.825 55.25) (width 0.4) (layer "F.Cu") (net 3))
 (segment (start 101.925 58.425) (end 100.625 58.425) (width 0.4) (layer "F.Cu") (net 3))
 (segment (start 100.625 58.425) (end 100.6 58.4) (width 0.4) (layer "F.Cu") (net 3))
 (segment (start 100.48 55.21) (end 101.91 55.21) (width 0.4) (layer "F.Cu") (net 3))
 (via (at 86.925 55.25) (size 0.6) (drill 0.3) (layers "F.Cu" "B.Cu") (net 3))
 (via (at 116.825 55.25) (size 0.6) (drill 0.3) (layers "F.Cu" "B.Cu") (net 3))
 (via (at 72.875 58.45) (size 0.6) (drill 0.3) (layers "F.Cu" "B.Cu") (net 3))
 (via (at 116.825 58.4) (size 0.6) (drill 0.3) (layers "F.Cu" "B.Cu") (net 3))
 (via (at 101.925 55.225) (size 0.6) (drill 0.3) (layers "F.Cu" "B.Cu") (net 3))
 (via (at 101.925 58.425) (size 0.6) (drill 0.3) (layers "F.Cu" "B.Cu") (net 3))
 (via (at 86.875 58.425) (size 0.6) (drill 0.3) (layers "F.Cu" "B.Cu") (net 3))
 (segment (start 72.875 58.45) (end 86.85 58.45) (width 0.4) (layer "B.Cu") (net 3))
 (segment (start 86.875 58.425) (end 86.875 55.3) (width 0.4) (layer "B.Cu") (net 3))
 (segment (start 86.875 58.425) (end 101.925 58.425) (width 0.4) (layer "B.Cu") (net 3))
 (segment (start 51.79 69.92) (end 51.79 82.62) (width 0.5) (layer "B.Cu") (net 3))
 (segment (start 116.825 58.4) (end 116.825 55.25) (width 0.4) (layer "B.Cu") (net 3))
 (segment (start 86.875 55.3) (end 86.925 55.25) (width 0.4) (layer "B.Cu") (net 3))
 (segment (start 54.33 67.38) (end 63.26 58.45) (width 0.4) (layer "B.Cu") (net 3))
 (segment (start 51.79 87.24) (end 51.79 82.62) (width 0.4) (layer "B.Cu") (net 3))
 (segment (start 84 97) (end 75.8 88.8) (width 0.4) (layer "B.Cu") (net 3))
 (segment (start 101.925 58.425) (end 101.925 55.875) (width 0.4) (layer "B.Cu") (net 3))
 (segment (start 131.575 58.4) (end 132.915 57.06) (width 0.4) (layer "B.Cu") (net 3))
 (segment (start 116.825 58.4) (end 131.575 58.4) (width 0.4) (layer "B.Cu") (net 3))
 (segment (start 63.26 58.45) (end 72.875 58.45) (width 0.4) (layer "B.Cu") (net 3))
 (segment (start 86.85 58.45) (end 86.875 58.425) (width 0.4) (layer "B.Cu") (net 3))
 (segment (start 75.8 88.8) (end 53.35 88.8) (width 0.4) (layer "B.Cu") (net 3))
 (segment (start 53.35 88.8) (end 51.79 87.24) (width 0.4) (layer "B.Cu") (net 3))
 (segment (start 101.925 55.875) (end 101.925 55.225) (width 0.5) (layer "B.Cu") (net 3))
 (segment (start 132.915 57.06) (end 137.5 57.06) (width 0.4) (layer "B.Cu") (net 3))
 (segment (start 54.33 67.38) (end 51.79 69.92) (width 0.5) (layer "B.Cu") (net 3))
 (segment (start 101.925 58.425) (end 116.8 58.425) (width 0.4) (layer "B.Cu") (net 3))
 (segment (start 116.8 58.425) (end 116.825 58.4) (width 0.4) (layer "B.Cu") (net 3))
 (segment (start 88.3957 59.1017) (end 90.2257 57.2717) (width 0.3) (layer "F.Cu") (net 14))
 (segment (start 100.6 56.57) (end 100.6 57.2717) (width 0.3) (layer "F.Cu") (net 14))
 (segment (start 90.2257 57.2717) (end 100.6 57.2717) (width 0.3) (layer "F.Cu") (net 14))
 (segment (start 84.45 59.1017) (end 88.3957 59.1017) (width 0.3) (layer "F.Cu") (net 14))
 (segment (start 84.45 58.4) (end 84.45 59.1017) (width 0.3) (layer "F.Cu") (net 14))
 (segment (start 84.3486 68.5492) (end 83.54 67.7406) (width 0.3) (layer "F.Cu") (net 6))
 (segment (start 85.9792 68.5492) (end 84.3486 68.5492) (width 0.3) (layer "F.Cu") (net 6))
 (segment (start 100.05 82.62) (end 85.9792 68.5492) (width 0.3) (layer "F.Cu") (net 6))
 (segment (start 75.9986 59.4438) (end 72.9223 59.4438) (width 0.3) (layer "F.Cu") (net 6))
 (segment (start 72.1882 58.1529) (end 72.8511 57.49) (width 0.3) (layer "F.Cu") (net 6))
 (segment (start 72.8511 57.49) (end 74.565 57.49) (width 0.3) (layer "F.Cu") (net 6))
 (segment (start 72.9223 59.4438) (end 72.1882 58.7097) (width 0.3) (layer "F.Cu") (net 6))
 (segment (start 83.54 66.9852) (end 75.9986 59.4438) (width 0.3) (layer "F.Cu") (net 6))
 (segment (start 72.1882 58.7097) (end 72.1882 58.1529) (width 0.3) (layer "F.Cu") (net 6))
 (segment (start 83.54 67.7406) (end 83.54 66.9852) (width 0.3) (layer "F.Cu") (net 6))
 (segment (start 108.2159 59.1017) (end 99.5 59.1017) (width 0.3) (layer "F.Cu") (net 13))
 (segment (start 115.55 57.2717) (end 110.0459 57.2717) (width 0.3) (layer "F.Cu") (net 13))
 (segment (start 115.55 56.57) (end 115.55 57.2717) (width 0.3) (layer "F.Cu") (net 13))
 (segment (start 99.5 58.4) (end 99.5 59.1017) (width 0.3) (layer "F.Cu") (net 13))
 (segment (start 110.0459 57.2717) (end 108.2159 59.1017) (width 0.3) (layer "F.Cu") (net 13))
 (segment (start 92 97) (end 93.4037 98.4037) (width 0.3) (layer "B.Cu") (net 10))
 (segment (start 113.7771 62.14) (end 137.5 62.14) (width 0.3) (layer "B.Cu") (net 10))
 (segment (start 82.27 93.2002) (end 85.8633 96.7935) (width 0.3) (layer "B.Cu") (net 10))
 (segment (start 85.8633 97.5029) (end 87.2152 98.8548) (width 0.3) (layer "B.Cu") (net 10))
 (segment (start 108.94 66.9771) (end 113.7771 62.14) (width 0.3) (layer "B.Cu") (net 10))
 (segment (start 90.1452 98.8548) (end 92 97) (width 0.3) (layer "B.Cu") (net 10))
 (segment (start 82.27 82.62) (end 82.27 93.2002) (width 0.3) (layer "B.Cu") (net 10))
 (segment (start 103.86 75.2955) (end 108.94 70.2155) (width 0.3) (layer "B.Cu") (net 10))
 (segment (start 96.5695 98.4037) (end 103.86 91.1132) (width 0.3) (layer "B.Cu") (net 10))
 (segment (start 87.2152 98.8548) (end 90.1452 98.8548) (width 0.3) (layer "B.Cu") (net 10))
 (segment (start 85.8633 96.7935) (end 85.8633 97.5029) (width 0.3) (layer "B.Cu") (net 10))
 (segment (start 93.4037 98.4037) (end 96.5695 98.4037) (width 0.3) (layer "B.Cu") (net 10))
 (segment (start 108.94 70.2155) (end 108.94 66.9771) (width 0.3) (layer "B.Cu") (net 10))
 (segment (start 103.86 91.1132) (end 103.86 75.2955) (width 0.3) (layer "B.Cu") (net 10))
 (segment (start 84.81 82.62) (end 85.9989 83.8089) (width 0.3) (layer "F.Cu") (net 11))
 (segment (start 101.32 83.0338) (end 101.32 82.2518) (width 0.3) (layer "F.Cu") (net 11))
 (segment (start 100.5449 83.8089) (end 101.32 83.0338) (width 0.3) (layer "F.Cu") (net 11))
 (segment (start 85.9989 83.8089) (end 100.5449 83.8089) (width 0.3) (layer "F.Cu") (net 11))
 (segment (start 118.8918 64.68) (end 137.5 64.68) (width 0.3) (layer "F.Cu") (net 11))
 (segment (start 101.32 82.2518) (end 118.8918 64.68) (width 0.3) (layer "F.Cu") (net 11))
 (segment (start 96 97) (end 94.6483 95.6483) (width 0.3) (layer "B.Cu") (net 11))
 (segment (start 88.7278 98.3531) (end 87.4229 98.3531) (width 0.3) (layer "B.Cu") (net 11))
 (segment (start 86.365 97.2952) (end 86.365 95.7186) (width 0.3) (layer "B.Cu") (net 11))
 (segment (start 87.4229 98.3531) (end 86.365 97.2952) (width 0.3) (layer "B.Cu") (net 11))
 (segment (start 86.365 95.7186) (end 84.81 94.1636) (width 0.3) (layer "B.Cu") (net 11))
 (segment (start 91.4326 95.6483) (end 88.7278 98.3531) (width 0.3) (layer "B.Cu") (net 11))
 (segment (start 94.6483 95.6483) (end 91.4326 95.6483) (width 0.3) (layer "B.Cu") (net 11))
 (segment (start 84.81 94.1636) (end 84.81 82.62) (width 0.3) (layer "B.Cu") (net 11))
 (segment (start 91.2502 60.9398) (end 136.1602 60.9398) (width 0.3) (layer "F.Cu") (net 9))
 (segment (start 136.1602 60.9398) (end 137.5 59.6) (width 0.3) (layer "F.Cu") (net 9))
 (segment (start 84.81 67.38) (end 91.2502 60.9398) (width 0.3) (layer "F.Cu") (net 9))
 (segment (start 86.08 68.65) (end 84.81 67.38) (width 0.3) (layer "B.Cu") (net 9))
 (segment (start 88 97) (end 88 96.2907) (width 0.3) (layer "B.Cu") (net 9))
 (segment (start 86.08 94.3707) (end 86.08 68.65) (width 0.3) (layer "B.Cu") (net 9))
 (segment (start 88 96.2907) (end 86.08 94.3707) (width 0.3) (layer "B.Cu") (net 9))
 (segment (start 102.6426 98.3574) (end 66.497 98.3574) (width 0.3) (layer "F.Cu") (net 1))
 (segment (start 104 97) (end 102.6426 98.3574) (width 0.3) (layer "F.Cu") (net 1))
 (segment (start 54.33 86.1904) (end 54.33 82.62) (width 0.3) (layer "F.Cu") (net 1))
 (segment (start 66.497 98.3574) (end 54.33 86.1904) (width 0.3) (layer "F.Cu") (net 1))
 (segment (start 104 97) (end 105.3547 98.3547) (width 0.3) (layer "B.Cu") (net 1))
 (segment (start 105.3547 98.3547) (end 123.2636 98.3547) (width 0.3) (layer "B.Cu") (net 1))
 (segment (start 123.2636 98.3547) (end 136.2983 85.32) (width 0.3) (layer "B.Cu") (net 1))
 (segment (start 137.5 85.32) (end 136.2983 85.32) (width 0.3) (layer "B.Cu") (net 1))
 (segment (start 108 97) (end 97.1746 86.1746) (width 0.3) (layer "F.Cu") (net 12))
 (segment (start 62.9646 86.1746) (end 59.41 82.62) (width 0.3) (layer "F.Cu") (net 12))
 (segment (start 117.14 87.86) (end 108 97) (width 0.3) (layer "F.Cu") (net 12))
 (segment (start 137.5 87.86) (end 117.14 87.86) (width 0.3) (layer "F.Cu") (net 12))
 (segment (start 97.1746 86.1746) (end 62.9646 86.1746) (width 0.3) (layer "F.Cu") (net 12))
 (segment (start 66.2194 84.3494) (end 104.9509 84.3494) (width 0.3) (layer "F.Cu") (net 4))
 (segment (start 116 97) (end 120.06 92.94) (width 0.3) (layer "F.Cu") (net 4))
 (segment (start 64.49 82.62) (end 66.2194 84.3494) (width 0.3) (layer "F.Cu") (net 4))
 (segment (start 120.06 92.94) (end 137.5 92.94) (width 0.3) (layer "F.Cu") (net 4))
 (segment (start 104.9509 84.3494) (end 105.0784 84.2219) (width 0.3) (layer "F.Cu") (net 4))
 (via (at 105.0784 84.2219) (size 0.6) (drill 0.3) (layers "F.Cu" "B.Cu") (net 4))
 (segment (start 116 95.1435) (end 105.0784 84.2219) (width 0.3) (layer "B.Cu") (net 4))
 (segment (start 116 97) (end 116 95.1435) (width 0.3) (layer "B.Cu") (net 4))
 (segment (start 112 97) (end 118.6 90.4) (width 0.3) (layer "F.Cu") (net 15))
 (segment (start 64.4035 85.0735) (end 104.9588 85.0735) (width 0.3) (layer "F.Cu") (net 15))
 (segment (start 118.6 90.4) (end 137.5 90.4) (width 0.3) (layer "F.Cu") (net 15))
 (segment (start 61.95 82.62) (end 64.4035 85.0735) (width 0.3) (layer "F.Cu") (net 15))
 (via (at 104.9588 85.0735) (size 0.6) (drill 0.3) (layers "F.Cu" "B.Cu") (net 15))
 (segment (start 112 97) (end 112 92.1147) (width 0.3) (layer "B.Cu") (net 15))
 (segment (start 112 92.1147) (end 104.9588 85.0735) (width 0.3) (layer "B.Cu") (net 15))
 (segment (start 135.98 97) (end 120 97) (width 0.3) (layer "F.Cu") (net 8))
 (segment (start 137.5 95.48) (end 135.98 97) (width 0.3) (layer "F.Cu") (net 8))
 (segment (start 120 77.17) (end 120 97) (width 0.3) (layer "B.Cu") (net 8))
 (segment (start 110.21 67.38) (end 120 77.17) (width 0.3) (layer "B.Cu") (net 8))
 (segment (start 85.55 57.2717) (end 80.5615 57.2717) (width 0.3) (layer "F.Cu") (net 7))
 (segment (start 85.55 56.57) (end 85.55 57.2717) (width 0.3) (layer "F.Cu") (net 7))
 (segment (start 80.5615 57.2717) (end 79.3932 58.44) (width 0.3) (layer "F.Cu") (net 7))
 (segment (start 79.3932 58.44) (end 76.84 58.44) (width 0.3) (layer "F.Cu") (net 7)))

